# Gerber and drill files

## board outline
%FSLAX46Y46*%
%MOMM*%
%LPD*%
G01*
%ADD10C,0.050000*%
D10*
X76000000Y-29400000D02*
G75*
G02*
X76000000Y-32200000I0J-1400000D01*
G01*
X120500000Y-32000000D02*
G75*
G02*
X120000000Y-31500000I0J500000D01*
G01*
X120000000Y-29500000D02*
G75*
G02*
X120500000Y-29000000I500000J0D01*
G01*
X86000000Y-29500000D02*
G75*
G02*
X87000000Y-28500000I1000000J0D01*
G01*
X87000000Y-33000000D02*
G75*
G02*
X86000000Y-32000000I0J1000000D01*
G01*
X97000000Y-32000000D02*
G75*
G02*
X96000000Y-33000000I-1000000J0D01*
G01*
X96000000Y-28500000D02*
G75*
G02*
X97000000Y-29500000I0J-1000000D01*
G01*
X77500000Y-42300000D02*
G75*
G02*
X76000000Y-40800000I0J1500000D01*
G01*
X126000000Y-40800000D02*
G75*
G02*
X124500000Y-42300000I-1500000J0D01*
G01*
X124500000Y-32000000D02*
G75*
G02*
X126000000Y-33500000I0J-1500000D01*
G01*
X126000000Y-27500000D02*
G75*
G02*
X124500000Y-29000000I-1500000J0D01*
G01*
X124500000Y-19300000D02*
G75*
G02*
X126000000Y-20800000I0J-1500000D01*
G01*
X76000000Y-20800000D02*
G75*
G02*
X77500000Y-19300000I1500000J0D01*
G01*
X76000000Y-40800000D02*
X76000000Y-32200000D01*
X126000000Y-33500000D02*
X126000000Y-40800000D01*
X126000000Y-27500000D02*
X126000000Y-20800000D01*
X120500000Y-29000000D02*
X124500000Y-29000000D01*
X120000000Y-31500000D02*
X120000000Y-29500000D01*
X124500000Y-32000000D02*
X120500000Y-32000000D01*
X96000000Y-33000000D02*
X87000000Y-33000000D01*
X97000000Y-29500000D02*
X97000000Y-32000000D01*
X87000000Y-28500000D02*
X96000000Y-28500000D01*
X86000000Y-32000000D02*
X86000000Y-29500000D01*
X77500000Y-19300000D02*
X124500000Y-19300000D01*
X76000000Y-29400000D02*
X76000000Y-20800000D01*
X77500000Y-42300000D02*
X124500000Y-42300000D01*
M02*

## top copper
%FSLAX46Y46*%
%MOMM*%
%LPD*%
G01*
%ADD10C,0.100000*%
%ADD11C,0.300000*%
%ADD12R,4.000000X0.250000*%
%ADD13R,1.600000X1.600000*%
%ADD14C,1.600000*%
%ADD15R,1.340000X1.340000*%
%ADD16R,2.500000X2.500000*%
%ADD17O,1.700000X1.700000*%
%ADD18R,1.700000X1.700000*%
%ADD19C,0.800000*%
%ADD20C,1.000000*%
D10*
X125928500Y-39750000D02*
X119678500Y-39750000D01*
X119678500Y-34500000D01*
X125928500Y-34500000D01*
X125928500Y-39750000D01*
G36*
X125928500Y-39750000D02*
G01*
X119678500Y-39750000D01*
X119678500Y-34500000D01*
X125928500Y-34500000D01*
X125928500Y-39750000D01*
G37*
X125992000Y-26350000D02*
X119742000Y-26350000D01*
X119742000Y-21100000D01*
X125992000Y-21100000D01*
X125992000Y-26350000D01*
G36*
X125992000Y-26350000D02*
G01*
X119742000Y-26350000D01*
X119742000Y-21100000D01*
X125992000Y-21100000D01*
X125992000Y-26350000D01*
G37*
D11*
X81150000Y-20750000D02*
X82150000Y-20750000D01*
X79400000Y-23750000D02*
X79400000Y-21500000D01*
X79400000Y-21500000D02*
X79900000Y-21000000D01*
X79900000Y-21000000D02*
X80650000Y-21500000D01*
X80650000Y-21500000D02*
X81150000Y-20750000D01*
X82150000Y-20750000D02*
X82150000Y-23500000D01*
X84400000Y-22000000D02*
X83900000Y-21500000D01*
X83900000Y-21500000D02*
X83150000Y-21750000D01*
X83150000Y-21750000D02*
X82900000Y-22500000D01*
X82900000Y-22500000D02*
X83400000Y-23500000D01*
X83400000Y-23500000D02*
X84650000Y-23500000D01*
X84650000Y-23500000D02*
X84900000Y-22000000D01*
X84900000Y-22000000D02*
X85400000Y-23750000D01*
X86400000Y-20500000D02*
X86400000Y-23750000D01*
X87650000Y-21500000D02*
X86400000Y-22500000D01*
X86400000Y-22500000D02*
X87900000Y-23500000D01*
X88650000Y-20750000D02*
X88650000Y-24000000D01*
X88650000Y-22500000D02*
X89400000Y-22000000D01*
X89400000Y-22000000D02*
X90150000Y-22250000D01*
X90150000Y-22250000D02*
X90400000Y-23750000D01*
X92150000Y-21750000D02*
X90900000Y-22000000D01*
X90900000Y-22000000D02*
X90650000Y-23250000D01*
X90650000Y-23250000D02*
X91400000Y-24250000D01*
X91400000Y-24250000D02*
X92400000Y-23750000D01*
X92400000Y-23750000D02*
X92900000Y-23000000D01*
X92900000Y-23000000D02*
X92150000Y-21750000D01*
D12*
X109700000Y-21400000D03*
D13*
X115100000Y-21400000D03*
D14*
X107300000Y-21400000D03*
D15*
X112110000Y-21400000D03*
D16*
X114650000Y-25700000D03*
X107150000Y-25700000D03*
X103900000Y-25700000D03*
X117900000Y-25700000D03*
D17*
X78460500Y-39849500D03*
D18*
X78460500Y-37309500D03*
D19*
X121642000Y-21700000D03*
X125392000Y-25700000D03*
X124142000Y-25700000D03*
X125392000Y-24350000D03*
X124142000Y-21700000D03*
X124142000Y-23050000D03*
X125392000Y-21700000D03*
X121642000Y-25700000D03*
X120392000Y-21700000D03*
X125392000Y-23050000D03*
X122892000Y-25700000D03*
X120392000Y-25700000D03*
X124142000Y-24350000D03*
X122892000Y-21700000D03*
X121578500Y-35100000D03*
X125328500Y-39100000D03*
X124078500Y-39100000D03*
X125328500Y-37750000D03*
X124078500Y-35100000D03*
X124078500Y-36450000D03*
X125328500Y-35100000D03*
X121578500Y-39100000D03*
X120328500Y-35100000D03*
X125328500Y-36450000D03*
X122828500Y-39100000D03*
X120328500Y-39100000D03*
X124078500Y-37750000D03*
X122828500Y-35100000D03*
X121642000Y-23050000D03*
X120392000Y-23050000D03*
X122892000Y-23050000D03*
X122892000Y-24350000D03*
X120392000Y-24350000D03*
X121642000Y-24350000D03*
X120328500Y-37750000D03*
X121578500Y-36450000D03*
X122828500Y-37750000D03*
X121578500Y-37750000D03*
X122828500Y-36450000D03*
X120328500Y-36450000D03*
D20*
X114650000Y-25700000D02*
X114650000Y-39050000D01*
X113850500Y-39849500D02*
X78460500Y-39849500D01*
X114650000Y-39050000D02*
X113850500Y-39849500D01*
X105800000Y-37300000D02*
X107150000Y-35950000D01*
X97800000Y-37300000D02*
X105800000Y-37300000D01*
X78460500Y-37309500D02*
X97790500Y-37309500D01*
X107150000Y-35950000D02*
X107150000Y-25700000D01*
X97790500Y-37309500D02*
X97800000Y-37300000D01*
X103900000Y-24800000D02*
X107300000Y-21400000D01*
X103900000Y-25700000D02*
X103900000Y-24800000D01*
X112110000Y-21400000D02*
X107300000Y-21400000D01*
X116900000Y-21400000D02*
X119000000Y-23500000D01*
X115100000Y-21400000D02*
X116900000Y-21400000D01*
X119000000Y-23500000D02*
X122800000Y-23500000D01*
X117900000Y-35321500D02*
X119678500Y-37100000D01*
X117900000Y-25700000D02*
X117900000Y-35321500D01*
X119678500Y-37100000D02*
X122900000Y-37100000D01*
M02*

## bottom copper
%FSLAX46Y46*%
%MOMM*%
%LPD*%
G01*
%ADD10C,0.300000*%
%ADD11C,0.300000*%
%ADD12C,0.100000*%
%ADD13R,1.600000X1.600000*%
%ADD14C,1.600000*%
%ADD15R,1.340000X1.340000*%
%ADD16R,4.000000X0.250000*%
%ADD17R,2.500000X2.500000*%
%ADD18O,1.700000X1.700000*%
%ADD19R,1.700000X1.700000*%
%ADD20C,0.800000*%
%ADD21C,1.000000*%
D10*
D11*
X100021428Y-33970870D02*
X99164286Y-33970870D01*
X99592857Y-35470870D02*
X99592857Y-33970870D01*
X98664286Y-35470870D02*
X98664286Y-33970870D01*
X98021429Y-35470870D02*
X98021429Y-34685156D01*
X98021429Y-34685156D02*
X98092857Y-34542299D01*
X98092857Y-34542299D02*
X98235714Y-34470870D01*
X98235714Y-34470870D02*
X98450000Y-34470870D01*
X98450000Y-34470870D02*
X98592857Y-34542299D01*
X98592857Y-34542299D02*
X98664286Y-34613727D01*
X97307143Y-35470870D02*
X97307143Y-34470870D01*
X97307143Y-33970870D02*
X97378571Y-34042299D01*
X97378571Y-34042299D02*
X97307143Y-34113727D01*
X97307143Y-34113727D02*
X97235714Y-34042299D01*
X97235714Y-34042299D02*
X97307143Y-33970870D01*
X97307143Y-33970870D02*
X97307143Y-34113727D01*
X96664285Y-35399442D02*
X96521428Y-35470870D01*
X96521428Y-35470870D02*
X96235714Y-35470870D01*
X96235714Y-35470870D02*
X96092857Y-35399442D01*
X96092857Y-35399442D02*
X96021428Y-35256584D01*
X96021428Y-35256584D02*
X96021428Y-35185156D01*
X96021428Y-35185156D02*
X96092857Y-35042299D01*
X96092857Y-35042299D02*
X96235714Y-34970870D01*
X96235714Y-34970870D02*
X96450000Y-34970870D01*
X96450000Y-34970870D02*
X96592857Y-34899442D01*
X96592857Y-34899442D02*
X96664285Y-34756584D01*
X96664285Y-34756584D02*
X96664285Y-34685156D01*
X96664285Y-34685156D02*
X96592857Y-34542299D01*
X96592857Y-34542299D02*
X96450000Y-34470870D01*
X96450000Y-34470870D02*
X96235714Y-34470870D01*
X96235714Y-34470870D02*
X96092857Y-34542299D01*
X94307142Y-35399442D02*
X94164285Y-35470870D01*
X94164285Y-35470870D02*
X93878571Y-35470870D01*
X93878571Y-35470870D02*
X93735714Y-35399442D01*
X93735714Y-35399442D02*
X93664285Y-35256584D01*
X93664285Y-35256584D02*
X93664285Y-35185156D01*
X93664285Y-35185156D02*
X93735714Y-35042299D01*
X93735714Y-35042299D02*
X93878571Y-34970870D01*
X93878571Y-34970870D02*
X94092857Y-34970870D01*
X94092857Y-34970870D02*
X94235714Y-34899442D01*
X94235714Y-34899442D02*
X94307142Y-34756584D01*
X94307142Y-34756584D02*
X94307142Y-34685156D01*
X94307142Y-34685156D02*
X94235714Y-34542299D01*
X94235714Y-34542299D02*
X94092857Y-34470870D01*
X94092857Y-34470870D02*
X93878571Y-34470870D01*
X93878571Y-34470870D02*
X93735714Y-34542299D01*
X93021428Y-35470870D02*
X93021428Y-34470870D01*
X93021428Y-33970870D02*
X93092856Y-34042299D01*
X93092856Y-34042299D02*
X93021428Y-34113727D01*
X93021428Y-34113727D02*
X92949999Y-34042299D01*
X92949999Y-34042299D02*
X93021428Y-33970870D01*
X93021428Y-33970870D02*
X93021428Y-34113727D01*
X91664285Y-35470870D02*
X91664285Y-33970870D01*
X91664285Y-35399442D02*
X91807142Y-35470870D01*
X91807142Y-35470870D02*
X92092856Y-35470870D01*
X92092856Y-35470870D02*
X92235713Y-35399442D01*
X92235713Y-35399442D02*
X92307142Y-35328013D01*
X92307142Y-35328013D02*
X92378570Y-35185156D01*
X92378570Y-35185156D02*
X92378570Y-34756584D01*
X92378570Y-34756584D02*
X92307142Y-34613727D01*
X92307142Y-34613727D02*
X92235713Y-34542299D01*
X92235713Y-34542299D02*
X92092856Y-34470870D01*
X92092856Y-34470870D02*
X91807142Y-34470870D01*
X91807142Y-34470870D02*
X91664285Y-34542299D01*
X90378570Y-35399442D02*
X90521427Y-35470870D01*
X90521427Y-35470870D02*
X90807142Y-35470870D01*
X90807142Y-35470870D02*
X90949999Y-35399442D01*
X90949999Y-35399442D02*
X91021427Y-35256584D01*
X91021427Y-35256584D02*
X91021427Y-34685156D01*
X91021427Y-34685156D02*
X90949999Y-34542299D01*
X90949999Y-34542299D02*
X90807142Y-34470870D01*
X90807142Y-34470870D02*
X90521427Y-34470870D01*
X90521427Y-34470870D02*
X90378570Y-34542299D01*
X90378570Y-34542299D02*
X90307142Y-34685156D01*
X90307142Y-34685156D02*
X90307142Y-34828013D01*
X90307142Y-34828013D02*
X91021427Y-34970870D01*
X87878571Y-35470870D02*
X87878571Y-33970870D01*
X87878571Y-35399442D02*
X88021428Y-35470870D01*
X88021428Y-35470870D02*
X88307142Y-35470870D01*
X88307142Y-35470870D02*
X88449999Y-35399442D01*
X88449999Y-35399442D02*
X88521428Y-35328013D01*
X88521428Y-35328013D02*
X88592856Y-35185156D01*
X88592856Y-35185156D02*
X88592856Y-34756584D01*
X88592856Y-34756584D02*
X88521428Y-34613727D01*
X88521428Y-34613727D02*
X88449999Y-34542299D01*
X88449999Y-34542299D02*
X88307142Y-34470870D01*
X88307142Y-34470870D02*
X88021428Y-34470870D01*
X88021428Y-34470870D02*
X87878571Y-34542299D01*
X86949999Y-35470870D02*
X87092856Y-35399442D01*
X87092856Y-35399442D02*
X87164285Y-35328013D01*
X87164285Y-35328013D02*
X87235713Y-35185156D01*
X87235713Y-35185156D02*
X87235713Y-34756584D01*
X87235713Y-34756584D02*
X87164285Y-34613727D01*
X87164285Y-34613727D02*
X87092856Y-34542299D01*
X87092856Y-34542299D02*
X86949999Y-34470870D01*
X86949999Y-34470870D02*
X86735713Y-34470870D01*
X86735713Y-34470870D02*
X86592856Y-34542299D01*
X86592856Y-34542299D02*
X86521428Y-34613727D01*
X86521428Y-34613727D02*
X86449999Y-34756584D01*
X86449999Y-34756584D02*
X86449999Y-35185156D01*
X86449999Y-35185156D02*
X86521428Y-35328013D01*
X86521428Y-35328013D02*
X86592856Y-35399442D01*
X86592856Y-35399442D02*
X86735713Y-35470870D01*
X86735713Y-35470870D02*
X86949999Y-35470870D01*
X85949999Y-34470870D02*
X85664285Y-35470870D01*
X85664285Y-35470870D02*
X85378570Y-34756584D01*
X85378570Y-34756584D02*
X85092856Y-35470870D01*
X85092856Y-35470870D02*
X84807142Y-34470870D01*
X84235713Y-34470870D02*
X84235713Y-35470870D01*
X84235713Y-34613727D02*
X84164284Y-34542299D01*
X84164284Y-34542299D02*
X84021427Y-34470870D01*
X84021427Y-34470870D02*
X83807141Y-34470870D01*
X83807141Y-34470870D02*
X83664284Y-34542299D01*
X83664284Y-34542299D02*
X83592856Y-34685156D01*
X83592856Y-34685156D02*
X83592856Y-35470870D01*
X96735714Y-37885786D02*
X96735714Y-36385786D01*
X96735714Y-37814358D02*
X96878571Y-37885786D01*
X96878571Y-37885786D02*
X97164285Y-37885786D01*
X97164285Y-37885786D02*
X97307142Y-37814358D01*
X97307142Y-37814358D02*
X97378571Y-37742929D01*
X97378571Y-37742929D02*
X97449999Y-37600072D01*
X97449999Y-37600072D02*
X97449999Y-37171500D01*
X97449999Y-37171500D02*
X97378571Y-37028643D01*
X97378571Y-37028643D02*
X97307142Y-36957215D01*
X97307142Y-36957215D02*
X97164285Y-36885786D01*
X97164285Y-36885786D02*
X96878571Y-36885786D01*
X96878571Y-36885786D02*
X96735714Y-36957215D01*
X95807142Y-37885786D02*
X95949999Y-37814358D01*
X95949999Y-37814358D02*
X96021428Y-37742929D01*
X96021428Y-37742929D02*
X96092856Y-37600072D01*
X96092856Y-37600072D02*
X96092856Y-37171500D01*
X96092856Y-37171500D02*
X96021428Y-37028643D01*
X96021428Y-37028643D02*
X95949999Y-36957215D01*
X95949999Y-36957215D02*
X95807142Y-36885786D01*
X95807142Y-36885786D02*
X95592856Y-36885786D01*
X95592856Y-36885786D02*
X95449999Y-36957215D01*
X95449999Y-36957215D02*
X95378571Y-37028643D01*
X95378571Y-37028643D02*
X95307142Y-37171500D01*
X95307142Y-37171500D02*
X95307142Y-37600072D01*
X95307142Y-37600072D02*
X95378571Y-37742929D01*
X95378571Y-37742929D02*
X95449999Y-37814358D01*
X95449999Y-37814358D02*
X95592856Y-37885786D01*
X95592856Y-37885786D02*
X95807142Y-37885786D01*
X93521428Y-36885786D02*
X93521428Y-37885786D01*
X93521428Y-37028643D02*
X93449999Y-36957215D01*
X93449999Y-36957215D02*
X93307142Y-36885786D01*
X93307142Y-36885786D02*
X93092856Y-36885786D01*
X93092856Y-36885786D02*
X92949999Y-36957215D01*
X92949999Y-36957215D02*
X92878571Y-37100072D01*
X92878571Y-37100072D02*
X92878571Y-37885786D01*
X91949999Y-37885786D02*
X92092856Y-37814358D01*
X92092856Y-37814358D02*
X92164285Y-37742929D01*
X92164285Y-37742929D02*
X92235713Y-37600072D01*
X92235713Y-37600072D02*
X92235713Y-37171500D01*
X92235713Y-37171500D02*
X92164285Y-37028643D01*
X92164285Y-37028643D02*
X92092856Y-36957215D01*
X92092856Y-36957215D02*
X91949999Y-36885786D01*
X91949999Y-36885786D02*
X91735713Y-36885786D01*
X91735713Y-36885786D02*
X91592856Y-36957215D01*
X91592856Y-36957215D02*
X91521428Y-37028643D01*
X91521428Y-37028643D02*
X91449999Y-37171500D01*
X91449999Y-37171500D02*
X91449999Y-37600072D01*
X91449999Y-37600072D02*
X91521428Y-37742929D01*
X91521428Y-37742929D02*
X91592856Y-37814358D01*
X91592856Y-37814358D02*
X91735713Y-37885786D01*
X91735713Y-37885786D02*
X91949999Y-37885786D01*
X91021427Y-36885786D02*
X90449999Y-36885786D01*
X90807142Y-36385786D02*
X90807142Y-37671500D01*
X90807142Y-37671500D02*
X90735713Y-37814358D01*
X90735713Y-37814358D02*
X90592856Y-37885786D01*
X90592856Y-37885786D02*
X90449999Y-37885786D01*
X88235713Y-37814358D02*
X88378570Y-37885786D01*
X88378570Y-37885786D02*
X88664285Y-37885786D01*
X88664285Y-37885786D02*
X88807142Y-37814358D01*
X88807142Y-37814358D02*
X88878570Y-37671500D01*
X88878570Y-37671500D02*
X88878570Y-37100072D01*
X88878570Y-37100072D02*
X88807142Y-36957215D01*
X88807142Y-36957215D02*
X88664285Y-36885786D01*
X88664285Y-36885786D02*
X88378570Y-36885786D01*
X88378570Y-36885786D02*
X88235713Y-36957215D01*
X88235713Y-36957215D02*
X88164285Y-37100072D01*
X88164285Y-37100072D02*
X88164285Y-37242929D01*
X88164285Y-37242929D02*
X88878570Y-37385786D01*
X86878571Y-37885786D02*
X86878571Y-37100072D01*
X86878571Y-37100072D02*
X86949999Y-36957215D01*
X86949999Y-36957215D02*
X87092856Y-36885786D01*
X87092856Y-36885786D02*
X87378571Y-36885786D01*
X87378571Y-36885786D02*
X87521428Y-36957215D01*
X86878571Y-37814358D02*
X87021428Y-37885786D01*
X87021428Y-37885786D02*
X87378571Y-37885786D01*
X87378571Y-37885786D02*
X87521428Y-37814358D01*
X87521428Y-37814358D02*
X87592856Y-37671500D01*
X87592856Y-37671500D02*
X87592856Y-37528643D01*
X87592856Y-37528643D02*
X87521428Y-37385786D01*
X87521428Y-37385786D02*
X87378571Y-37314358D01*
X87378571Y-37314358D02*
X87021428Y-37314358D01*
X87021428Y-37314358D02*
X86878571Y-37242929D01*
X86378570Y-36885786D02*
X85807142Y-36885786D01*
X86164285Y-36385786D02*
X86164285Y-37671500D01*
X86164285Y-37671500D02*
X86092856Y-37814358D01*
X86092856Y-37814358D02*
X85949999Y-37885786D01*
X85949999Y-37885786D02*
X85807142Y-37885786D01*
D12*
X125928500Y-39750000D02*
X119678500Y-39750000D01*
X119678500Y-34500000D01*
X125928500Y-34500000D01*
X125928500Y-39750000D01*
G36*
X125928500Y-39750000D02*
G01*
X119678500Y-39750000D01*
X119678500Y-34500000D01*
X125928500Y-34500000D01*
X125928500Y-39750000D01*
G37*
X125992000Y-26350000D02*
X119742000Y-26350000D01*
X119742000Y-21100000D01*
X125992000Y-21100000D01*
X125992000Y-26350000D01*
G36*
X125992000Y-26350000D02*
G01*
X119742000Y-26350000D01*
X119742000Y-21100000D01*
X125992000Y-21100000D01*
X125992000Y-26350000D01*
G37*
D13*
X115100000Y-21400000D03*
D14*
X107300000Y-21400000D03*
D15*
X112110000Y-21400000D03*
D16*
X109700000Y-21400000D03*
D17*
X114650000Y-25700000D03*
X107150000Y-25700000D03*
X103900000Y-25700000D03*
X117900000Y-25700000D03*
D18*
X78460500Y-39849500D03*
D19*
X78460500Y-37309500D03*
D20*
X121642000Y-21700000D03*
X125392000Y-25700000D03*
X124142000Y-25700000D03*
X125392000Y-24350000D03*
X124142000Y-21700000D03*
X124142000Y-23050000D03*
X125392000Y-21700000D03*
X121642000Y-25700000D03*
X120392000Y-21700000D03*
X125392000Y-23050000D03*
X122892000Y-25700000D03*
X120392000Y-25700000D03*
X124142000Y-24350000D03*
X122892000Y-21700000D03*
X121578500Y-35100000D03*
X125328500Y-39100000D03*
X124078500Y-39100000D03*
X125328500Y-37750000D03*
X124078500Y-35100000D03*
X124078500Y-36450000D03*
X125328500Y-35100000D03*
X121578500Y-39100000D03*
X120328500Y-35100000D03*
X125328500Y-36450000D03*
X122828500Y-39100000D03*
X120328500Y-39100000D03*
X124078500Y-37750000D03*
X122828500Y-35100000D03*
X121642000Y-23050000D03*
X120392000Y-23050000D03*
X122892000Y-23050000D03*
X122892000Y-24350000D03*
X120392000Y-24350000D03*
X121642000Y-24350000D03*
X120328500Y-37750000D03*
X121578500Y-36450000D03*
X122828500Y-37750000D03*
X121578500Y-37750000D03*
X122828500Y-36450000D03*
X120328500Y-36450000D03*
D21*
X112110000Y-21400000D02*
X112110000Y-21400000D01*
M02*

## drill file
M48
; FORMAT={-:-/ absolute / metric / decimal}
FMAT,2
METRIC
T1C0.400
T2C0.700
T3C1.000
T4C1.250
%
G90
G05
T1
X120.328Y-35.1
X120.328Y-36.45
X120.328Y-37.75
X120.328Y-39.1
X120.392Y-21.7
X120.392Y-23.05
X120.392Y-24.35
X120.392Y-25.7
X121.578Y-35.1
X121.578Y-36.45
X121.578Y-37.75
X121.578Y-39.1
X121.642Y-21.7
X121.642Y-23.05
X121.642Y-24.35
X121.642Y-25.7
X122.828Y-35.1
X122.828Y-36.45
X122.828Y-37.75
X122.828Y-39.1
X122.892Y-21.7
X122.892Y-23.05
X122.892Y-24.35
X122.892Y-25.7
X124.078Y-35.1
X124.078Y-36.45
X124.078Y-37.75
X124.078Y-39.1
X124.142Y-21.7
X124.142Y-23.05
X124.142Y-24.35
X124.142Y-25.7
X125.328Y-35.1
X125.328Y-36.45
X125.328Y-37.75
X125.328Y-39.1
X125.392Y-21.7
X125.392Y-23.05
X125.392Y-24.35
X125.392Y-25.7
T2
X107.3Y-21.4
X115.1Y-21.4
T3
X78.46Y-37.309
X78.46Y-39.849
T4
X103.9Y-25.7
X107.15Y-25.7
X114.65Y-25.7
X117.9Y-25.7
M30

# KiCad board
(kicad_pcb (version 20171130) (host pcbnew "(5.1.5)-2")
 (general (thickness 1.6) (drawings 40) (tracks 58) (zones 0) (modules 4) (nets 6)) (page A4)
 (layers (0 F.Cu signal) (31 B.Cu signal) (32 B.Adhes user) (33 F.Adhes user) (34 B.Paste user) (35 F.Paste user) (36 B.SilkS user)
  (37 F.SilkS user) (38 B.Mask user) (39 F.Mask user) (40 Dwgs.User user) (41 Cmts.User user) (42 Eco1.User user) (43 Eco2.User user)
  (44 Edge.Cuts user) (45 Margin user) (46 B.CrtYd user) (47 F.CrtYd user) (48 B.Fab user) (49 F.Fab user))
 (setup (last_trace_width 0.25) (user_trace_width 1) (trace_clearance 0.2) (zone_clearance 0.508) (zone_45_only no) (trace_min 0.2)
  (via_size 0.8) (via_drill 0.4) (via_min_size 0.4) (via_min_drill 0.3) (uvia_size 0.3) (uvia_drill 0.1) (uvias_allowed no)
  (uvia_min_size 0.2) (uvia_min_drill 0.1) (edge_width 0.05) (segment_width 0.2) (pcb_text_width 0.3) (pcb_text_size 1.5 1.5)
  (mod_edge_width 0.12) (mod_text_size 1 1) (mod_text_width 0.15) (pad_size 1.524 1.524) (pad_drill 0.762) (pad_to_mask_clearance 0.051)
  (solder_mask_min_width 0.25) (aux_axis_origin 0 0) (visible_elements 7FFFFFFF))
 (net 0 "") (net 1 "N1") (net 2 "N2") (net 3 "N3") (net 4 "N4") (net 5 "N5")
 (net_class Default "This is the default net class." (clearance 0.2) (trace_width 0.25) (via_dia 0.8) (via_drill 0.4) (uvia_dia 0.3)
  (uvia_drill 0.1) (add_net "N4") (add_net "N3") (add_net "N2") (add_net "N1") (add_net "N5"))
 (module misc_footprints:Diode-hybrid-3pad (layer F.Cu) (at 111.2 21.4)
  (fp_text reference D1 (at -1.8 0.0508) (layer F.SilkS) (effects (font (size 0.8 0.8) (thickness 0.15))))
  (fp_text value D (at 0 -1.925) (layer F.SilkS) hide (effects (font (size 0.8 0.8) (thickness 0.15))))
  (pad 2 smd rect (at -1.5 0) (size 4 0.25) (layers F.Cu) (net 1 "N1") (solder_mask_margin -999))
  (pad 1 thru_hole rect (at 3.9 0) (size 1.6 1.6) (drill 0.7) (layers *.Cu *.Mask F.SilkS) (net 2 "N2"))
  (pad 2 thru_hole circle (at -3.9 0) (size 1.6 1.6) (drill 0.7) (layers *.Cu *.Mask F.SilkS) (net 1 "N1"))
  (pad 2 smd rect (at 0.91 0) (size 1.34 1.34) (layers F.Cu F.Paste F.Mask) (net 1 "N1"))
  (pad 2 smd rect (at 0.91 0) (size 1.34 1.34) (layers B.Cu B.Paste B.Mask) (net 1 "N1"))
  (pad 2 smd rect (at -1.5 0) (size 4 0.25) (layers B.Cu) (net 1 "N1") (solder_mask_margin -999)))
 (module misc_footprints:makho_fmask (layer F.Cu) (at 85.9 22.5)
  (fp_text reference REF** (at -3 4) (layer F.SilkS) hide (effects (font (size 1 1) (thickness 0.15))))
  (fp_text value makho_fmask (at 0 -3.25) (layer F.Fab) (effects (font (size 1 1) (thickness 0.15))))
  (fp_line (start -4.75 -1.75) (end -3.75 -1.75) (layer F.Cu) (width 0.3))
  (fp_line (start -6.5 1.25) (end -6.5 -1) (layer F.Cu) (width 0.3))
  (fp_line (start -6.5 -1) (end -6 -1.5) (layer F.Cu) (width 0.3))
  (fp_line (start -6 -1.5) (end -5.25 -1) (layer F.Cu) (width 0.3))
  (fp_line (start -5.25 -1) (end -4.75 -1.75) (layer F.Cu) (width 0.3))
  (fp_line (start -3.75 -1.75) (end -3.75 1) (layer F.Cu) (width 0.3))
  (fp_line (start -1.5 -0.5) (end -2 -1) (layer F.Cu) (width 0.3))
  (fp_line (start -2 -1) (end -2.75 -0.75) (layer F.Cu) (width 0.3))
  (fp_line (start -2.75 -0.75) (end -3 0) (layer F.Cu) (width 0.3)) (fp_line (start -3 0) (end -2.5 1) (layer F.Cu) (width 0.3))
  (fp_line (start -2.5 1) (end -1.25 1) (layer F.Cu) (width 0.3))
  (fp_line (start -1.25 1) (end -1 -0.5) (layer F.Cu) (width 0.3))
  (fp_line (start -1 -0.5) (end -0.5 1.25) (layer F.Cu) (width 0.3))
  (fp_line (start 0.5 -2) (end 0.5 1.25) (layer F.Cu) (width 0.3))
  (fp_line (start 1.75 -1) (end 0.5 0) (layer F.Cu) (width 0.3)) (fp_line (start 0.5 0) (end 2 1) (layer F.Cu) (width 0.3))
  (fp_line (start 2.75 -1.75) (end 2.75 1.5) (layer F.Cu) (width 0.3))
  (fp_line (start 2.75 0) (end 3.5 -0.5) (layer F.Cu) (width 0.3))
  (fp_line (start 3.5 -0.5) (end 4.25 -0.25) (layer F.Cu) (width 0.3))
  (fp_line (start 4.25 -0.25) (end 4.5 1.25) (layer F.Cu) (width 0.3))
  (fp_line (start 6.25 -0.75) (end 5 -0.5) (layer F.Cu) (width 0.3))
  (fp_line (start 5 -0.5) (end 4.75 0.75) (layer F.Cu) (width 0.3))
  (fp_line (start 4.75 0.75) (end 5.5 1.75) (layer F.Cu) (width 0.3))
  (fp_line (start 5.5 1.75) (end 6.5 1.25) (layer F.Cu) (width 0.3))
  (fp_line (start 6.5 1.25) (end 7 0.5) (layer F.Cu) (width 0.3))
  (fp_line (start 7 0.5) (end 6.25 -0.75) (layer F.Cu) (width 0.3)))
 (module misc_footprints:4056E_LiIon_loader (layer F.Cu) (at 110.9 36.7 90)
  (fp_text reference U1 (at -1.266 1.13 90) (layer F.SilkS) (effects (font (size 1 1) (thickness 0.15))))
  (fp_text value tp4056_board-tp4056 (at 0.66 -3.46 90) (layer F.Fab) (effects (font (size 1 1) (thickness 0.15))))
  (pad 4 thru_hole rect (at 11 3.75 90) (size 2.5 2.5) (drill 1.25) (layers *.Cu *.Mask F.SilkS) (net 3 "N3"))
  (pad 3 thru_hole rect (at 11 -3.75 90) (size 2.5 2.5) (drill 1.25) (layers *.Cu *.Mask F.SilkS) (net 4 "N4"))
  (pad 5 thru_hole rect (at 11 -7 90) (size 2.5 2.5) (drill 1.25) (layers *.Cu *.Mask F.SilkS) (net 1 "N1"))
  (pad 6 thru_hole rect (at 11 7 90) (size 2.5 2.5) (drill 1.25) (layers *.Cu *.Mask F.SilkS) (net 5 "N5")))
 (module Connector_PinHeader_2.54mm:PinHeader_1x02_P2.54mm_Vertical (layer F.Cu) (at 78.4605 37.3095)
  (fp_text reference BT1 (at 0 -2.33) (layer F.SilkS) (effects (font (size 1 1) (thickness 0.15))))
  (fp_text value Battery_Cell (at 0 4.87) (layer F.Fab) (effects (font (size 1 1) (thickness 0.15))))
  (pad 2 thru_hole oval (at 0 2.54) (size 1.7 1.7) (drill 1) (layers *.Cu *.Mask) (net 3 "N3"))
  (pad 1 thru_hole rect (at 0 0) (size 1.7 1.7) (drill 1) (layers *.Cu *.Mask) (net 4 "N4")))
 (gr_arc (start 76 30.8) (end 76 32.2) (angle -180) (layer Edge.Cuts) (width 0.05))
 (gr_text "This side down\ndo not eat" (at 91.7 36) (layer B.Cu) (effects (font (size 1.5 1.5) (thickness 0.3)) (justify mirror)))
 (gr_poly (pts (xy 125.9285 39.75) (xy 119.6785 39.75) (xy 119.6785 34.5) (xy 125.9285 34.5)) (layer B.Cu) (width 0.1))
 (gr_poly (pts (xy 125.9285 39.75) (xy 119.6785 39.75) (xy 119.6785 34.5) (xy 125.9285 34.5)) (layer F.Cu) (width 0.1))
 (gr_poly (pts (xy 125.992 26.35) (xy 119.742 26.35) (xy 119.742 21.1) (xy 125.992 21.1)) (layer B.Cu) (width 0.1))
 (gr_arc (start 120.5 31.5) (end 120 31.5) (angle -90) (layer Edge.Cuts) (width 0.05))
 (gr_arc (start 120.5 29.5) (end 120.5 29) (angle -90) (layer Edge.Cuts) (width 0.05))
 (gr_poly (pts (xy 125.992 26.35) (xy 119.742 26.35) (xy 119.742 21.1) (xy 125.992 21.1)) (layer F.Cu) (width 0.1))
 (gr_arc (start 87 29.5) (end 87 28.5) (angle -90) (layer Edge.Cuts) (width 0.05))
 (gr_arc (start 87 32) (end 86 32) (angle -90) (layer Edge.Cuts) (width 0.05))
 (gr_arc (start 96 32) (end 96 33) (angle -90) (layer Edge.Cuts) (width 0.05))
 (gr_arc (start 96 29.5) (end 97 29.5) (angle -90) (layer Edge.Cuts) (width 0.05))
 (gr_arc (start 77.5 40.8) (end 76 40.8) (angle -90) (layer Edge.Cuts) (width 0.05))
 (gr_arc (start 124.5 40.8) (end 124.5 42.3) (angle -90) (layer Edge.Cuts) (width 0.05))
 (gr_arc (start 124.5 33.5) (end 126 33.5) (angle -90) (layer Edge.Cuts) (width 0.05))
 (gr_arc (start 124.5 27.5) (end 124.5 29) (angle -90) (layer Edge.Cuts) (width 0.05))
 (gr_arc (start 124.5 20.8) (end 126 20.8) (angle -90) (layer Edge.Cuts) (width 0.05))
 (gr_arc (start 77.5 20.8) (end 77.5 19.3) (angle -90) (layer Edge.Cuts) (width 0.05))
 (gr_line (start 76 40.8) (end 76 32.2) (layer Edge.Cuts) (width 0.05))
 (gr_line (start 126 33.5) (end 126 40.8) (layer Edge.Cuts) (width 0.05))
 (gr_line (start 126 27.5) (end 126 20.8) (layer Edge.Cuts) (width 0.05))
 (gr_line (start 120.5 29) (end 124.5 29) (layer Edge.Cuts) (width 0.05))
 (gr_line (start 120 31.5) (end 120 29.5) (layer Edge.Cuts) (width 0.05))
 (gr_line (start 124.5 32) (end 120.5 32) (layer Edge.Cuts) (width 0.05))
 (gr_line (start 96 33) (end 87 33) (layer Edge.Cuts) (width 0.05))
 (gr_line (start 97 29.5) (end 97 32) (layer Edge.Cuts) (width 0.05))
 (gr_line (start 87 28.5) (end 96 28.5) (layer Edge.Cuts) (width 0.05))
 (gr_line (start 86 32) (end 86 29.5) (layer Edge.Cuts) (width 0.05))
 (gr_line (start 77.5 19.3) (end 124.5 19.3) (layer Edge.Cuts) (width 0.05))
 (gr_line (start 76 29.4) (end 76 20.8) (layer Edge.Cuts) (width 0.05))
 (gr_line (start 77.5 42.3) (end 124.5 42.3) (layer Edge.Cuts) (width 0.05))
 (via (at 121.642 21.7) (size 0.8) (drill 0.4) (layers F.Cu B.Cu) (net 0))
 (via (at 125.392 25.7) (size 0.8) (drill 0.4) (layers F.Cu B.Cu) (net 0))
 (via (at 124.142 25.7) (size 0.8) (drill 0.4) (layers F.Cu B.Cu) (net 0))
 (via (at 125.392 24.35) (size 0.8) (drill 0.4) (layers F.Cu B.Cu) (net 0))
 (via (at 124.142 21.7) (size 0.8) (drill 0.4) (layers F.Cu B.Cu) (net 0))
 (via (at 124.142 23.05) (size 0.8) (drill 0.4) (layers F.Cu B.Cu) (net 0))
 (via (at 125.392 21.7) (size 0.8) (drill 0.4) (layers F.Cu B.Cu) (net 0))
 (via (at 121.642 25.7) (size 0.8) (drill 0.4) (layers F.Cu B.Cu) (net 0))
 (via (at 120.392 21.7) (size 0.8) (drill 0.4) (layers F.Cu B.Cu) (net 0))
 (via (at 125.392 23.05) (size 0.8) (drill 0.4) (layers F.Cu B.Cu) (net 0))
 (via (at 122.892 25.7) (size 0.8) (drill 0.4) (layers F.Cu B.Cu) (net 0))
 (via (at 120.392 25.7) (size 0.8) (drill 0.4) (layers F.Cu B.Cu) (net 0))
 (via (at 124.142 24.35) (size 0.8) (drill 0.4) (layers F.Cu B.Cu) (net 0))
 (via (at 122.892 21.7) (size 0.8) (drill 0.4) (layers F.Cu B.Cu) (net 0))
 (via (at 121.5785 35.1) (size 0.8) (drill 0.4) (layers F.Cu B.Cu) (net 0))
 (via (at 125.3285 39.1) (size 0.8) (drill 0.4) (layers F.Cu B.Cu) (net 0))
 (via (at 124.0785 39.1) (size 0.8) (drill 0.4) (layers F.Cu B.Cu) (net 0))
 (via (at 125.3285 37.75) (size 0.8) (drill 0.4) (layers F.Cu B.Cu) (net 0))
 (via (at 124.0785 35.1) (size 0.8) (drill 0.4) (layers F.Cu B.Cu) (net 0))
 (via (at 124.0785 36.45) (size 0.8) (drill 0.4) (layers F.Cu B.Cu) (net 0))
 (via (at 125.3285 35.1) (size 0.8) (drill 0.4) (layers F.Cu B.Cu) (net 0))
 (via (at 121.5785 39.1) (size 0.8) (drill 0.4) (layers F.Cu B.Cu) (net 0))
 (via (at 120.3285 35.1) (size 0.8) (drill 0.4) (layers F.Cu B.Cu) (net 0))
 (via (at 125.3285 36.45) (size 0.8) (drill 0.4) (layers F.Cu B.Cu) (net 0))
 (via (at 122.8285 39.1) (size 0.8) (drill 0.4) (layers F.Cu B.Cu) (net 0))
 (via (at 120.3285 39.1) (size 0.8) (drill 0.4) (layers F.Cu B.Cu) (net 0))
 (via (at 124.0785 37.75) (size 0.8) (drill 0.4) (layers F.Cu B.Cu) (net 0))
 (via (at 122.8285 35.1) (size 0.8) (drill 0.4) (layers F.Cu B.Cu) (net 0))
 (segment (start 114.65 25.7) (end 114.65 39.05) (width 1) (layer F.Cu) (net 3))
 (segment (start 113.8505 39.8495) (end 78.4605 39.8495) (width 1) (layer F.Cu) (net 3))
 (segment (start 114.65 39.05) (end 113.8505 39.8495) (width 1) (layer F.Cu) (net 3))
 (segment (start 105.8 37.3) (end 107.15 35.95) (width 1) (layer F.Cu) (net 4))
 (segment (start 97.8 37.3) (end 105.8 37.3) (width 1) (layer F.Cu) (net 4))
 (segment (start 78.4605 37.3095) (end 97.7905 37.3095) (width 1) (layer F.Cu) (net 4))
 (segment (start 107.15 35.95) (end 107.15 25.7) (width 1) (layer F.Cu) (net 4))
 (segment (start 97.7905 37.3095) (end 97.8 37.3) (width 1) (layer F.Cu) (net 4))
 (segment (start 103.9 24.8) (end 107.3 21.4) (width 1) (layer F.Cu) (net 1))
 (segment (start 103.9 25.7) (end 103.9 24.8) (width 1) (layer F.Cu) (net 1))
 (segment (start 112.11 21.4) (end 112.11 21.4) (width 1) (layer B.Cu) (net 1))
 (segment (start 112.11 21.4) (end 107.3 21.4) (width 1) (layer F.Cu) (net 1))
 (via (at 121.642 23.05) (size 0.8) (drill 0.4) (layers F.Cu B.Cu) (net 2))
 (via (at 120.392 23.05) (size 0.8) (drill 0.4) (layers F.Cu B.Cu) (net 2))
 (via (at 122.892 23.05) (size 0.8) (drill 0.4) (layers F.Cu B.Cu) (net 2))
 (via (at 122.892 24.35) (size 0.8) (drill 0.4) (layers F.Cu B.Cu) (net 2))
 (via (at 120.392 24.35) (size 0.8) (drill 0.4) (layers F.Cu B.Cu) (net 2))
 (via (at 121.642 24.35) (size 0.8) (drill 0.4) (layers F.Cu B.Cu) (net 2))
 (segment (start 116.9 21.4) (end 119 23.5) (width 1) (layer F.Cu) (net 2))
 (segment (start 115.1 21.4) (end 116.9 21.4) (width 1) (layer F.Cu) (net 2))
 (segment (start 119 23.5) (end 122.8 23.5) (width 1) (layer F.Cu) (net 2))
 (via (at 120.3285 37.75) (size 0.8) (drill 0.4) (layers F.Cu B.Cu) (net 5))
 (via (at 121.5785 36.45) (size 0.8) (drill 0.4) (layers F.Cu B.Cu) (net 5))
 (via (at 122.8285 37.75) (size 0.8) (drill 0.4) (layers F.Cu B.Cu) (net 5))
 (via (at 121.5785 37.75) (size 0.8) (drill 0.4) (layers F.Cu B.Cu) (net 5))
 (via (at 122.8285 36.45) (size 0.8) (drill 0.4) (layers F.Cu B.Cu) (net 5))
 (via (at 120.3285 36.45) (size 0.8) (drill 0.4) (layers F.Cu B.Cu) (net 5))
 (segment (start 117.9 35.3215) (end 119.6785 37.1) (width 1) (layer F.Cu) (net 5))
 (segment (start 117.9 25.7) (end 117.9 35.3215) (width 1) (layer F.Cu) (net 5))
 (segment (start 119.6785 37.1) (end 122.9 37.1) (width 1) (layer F.Cu) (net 5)))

